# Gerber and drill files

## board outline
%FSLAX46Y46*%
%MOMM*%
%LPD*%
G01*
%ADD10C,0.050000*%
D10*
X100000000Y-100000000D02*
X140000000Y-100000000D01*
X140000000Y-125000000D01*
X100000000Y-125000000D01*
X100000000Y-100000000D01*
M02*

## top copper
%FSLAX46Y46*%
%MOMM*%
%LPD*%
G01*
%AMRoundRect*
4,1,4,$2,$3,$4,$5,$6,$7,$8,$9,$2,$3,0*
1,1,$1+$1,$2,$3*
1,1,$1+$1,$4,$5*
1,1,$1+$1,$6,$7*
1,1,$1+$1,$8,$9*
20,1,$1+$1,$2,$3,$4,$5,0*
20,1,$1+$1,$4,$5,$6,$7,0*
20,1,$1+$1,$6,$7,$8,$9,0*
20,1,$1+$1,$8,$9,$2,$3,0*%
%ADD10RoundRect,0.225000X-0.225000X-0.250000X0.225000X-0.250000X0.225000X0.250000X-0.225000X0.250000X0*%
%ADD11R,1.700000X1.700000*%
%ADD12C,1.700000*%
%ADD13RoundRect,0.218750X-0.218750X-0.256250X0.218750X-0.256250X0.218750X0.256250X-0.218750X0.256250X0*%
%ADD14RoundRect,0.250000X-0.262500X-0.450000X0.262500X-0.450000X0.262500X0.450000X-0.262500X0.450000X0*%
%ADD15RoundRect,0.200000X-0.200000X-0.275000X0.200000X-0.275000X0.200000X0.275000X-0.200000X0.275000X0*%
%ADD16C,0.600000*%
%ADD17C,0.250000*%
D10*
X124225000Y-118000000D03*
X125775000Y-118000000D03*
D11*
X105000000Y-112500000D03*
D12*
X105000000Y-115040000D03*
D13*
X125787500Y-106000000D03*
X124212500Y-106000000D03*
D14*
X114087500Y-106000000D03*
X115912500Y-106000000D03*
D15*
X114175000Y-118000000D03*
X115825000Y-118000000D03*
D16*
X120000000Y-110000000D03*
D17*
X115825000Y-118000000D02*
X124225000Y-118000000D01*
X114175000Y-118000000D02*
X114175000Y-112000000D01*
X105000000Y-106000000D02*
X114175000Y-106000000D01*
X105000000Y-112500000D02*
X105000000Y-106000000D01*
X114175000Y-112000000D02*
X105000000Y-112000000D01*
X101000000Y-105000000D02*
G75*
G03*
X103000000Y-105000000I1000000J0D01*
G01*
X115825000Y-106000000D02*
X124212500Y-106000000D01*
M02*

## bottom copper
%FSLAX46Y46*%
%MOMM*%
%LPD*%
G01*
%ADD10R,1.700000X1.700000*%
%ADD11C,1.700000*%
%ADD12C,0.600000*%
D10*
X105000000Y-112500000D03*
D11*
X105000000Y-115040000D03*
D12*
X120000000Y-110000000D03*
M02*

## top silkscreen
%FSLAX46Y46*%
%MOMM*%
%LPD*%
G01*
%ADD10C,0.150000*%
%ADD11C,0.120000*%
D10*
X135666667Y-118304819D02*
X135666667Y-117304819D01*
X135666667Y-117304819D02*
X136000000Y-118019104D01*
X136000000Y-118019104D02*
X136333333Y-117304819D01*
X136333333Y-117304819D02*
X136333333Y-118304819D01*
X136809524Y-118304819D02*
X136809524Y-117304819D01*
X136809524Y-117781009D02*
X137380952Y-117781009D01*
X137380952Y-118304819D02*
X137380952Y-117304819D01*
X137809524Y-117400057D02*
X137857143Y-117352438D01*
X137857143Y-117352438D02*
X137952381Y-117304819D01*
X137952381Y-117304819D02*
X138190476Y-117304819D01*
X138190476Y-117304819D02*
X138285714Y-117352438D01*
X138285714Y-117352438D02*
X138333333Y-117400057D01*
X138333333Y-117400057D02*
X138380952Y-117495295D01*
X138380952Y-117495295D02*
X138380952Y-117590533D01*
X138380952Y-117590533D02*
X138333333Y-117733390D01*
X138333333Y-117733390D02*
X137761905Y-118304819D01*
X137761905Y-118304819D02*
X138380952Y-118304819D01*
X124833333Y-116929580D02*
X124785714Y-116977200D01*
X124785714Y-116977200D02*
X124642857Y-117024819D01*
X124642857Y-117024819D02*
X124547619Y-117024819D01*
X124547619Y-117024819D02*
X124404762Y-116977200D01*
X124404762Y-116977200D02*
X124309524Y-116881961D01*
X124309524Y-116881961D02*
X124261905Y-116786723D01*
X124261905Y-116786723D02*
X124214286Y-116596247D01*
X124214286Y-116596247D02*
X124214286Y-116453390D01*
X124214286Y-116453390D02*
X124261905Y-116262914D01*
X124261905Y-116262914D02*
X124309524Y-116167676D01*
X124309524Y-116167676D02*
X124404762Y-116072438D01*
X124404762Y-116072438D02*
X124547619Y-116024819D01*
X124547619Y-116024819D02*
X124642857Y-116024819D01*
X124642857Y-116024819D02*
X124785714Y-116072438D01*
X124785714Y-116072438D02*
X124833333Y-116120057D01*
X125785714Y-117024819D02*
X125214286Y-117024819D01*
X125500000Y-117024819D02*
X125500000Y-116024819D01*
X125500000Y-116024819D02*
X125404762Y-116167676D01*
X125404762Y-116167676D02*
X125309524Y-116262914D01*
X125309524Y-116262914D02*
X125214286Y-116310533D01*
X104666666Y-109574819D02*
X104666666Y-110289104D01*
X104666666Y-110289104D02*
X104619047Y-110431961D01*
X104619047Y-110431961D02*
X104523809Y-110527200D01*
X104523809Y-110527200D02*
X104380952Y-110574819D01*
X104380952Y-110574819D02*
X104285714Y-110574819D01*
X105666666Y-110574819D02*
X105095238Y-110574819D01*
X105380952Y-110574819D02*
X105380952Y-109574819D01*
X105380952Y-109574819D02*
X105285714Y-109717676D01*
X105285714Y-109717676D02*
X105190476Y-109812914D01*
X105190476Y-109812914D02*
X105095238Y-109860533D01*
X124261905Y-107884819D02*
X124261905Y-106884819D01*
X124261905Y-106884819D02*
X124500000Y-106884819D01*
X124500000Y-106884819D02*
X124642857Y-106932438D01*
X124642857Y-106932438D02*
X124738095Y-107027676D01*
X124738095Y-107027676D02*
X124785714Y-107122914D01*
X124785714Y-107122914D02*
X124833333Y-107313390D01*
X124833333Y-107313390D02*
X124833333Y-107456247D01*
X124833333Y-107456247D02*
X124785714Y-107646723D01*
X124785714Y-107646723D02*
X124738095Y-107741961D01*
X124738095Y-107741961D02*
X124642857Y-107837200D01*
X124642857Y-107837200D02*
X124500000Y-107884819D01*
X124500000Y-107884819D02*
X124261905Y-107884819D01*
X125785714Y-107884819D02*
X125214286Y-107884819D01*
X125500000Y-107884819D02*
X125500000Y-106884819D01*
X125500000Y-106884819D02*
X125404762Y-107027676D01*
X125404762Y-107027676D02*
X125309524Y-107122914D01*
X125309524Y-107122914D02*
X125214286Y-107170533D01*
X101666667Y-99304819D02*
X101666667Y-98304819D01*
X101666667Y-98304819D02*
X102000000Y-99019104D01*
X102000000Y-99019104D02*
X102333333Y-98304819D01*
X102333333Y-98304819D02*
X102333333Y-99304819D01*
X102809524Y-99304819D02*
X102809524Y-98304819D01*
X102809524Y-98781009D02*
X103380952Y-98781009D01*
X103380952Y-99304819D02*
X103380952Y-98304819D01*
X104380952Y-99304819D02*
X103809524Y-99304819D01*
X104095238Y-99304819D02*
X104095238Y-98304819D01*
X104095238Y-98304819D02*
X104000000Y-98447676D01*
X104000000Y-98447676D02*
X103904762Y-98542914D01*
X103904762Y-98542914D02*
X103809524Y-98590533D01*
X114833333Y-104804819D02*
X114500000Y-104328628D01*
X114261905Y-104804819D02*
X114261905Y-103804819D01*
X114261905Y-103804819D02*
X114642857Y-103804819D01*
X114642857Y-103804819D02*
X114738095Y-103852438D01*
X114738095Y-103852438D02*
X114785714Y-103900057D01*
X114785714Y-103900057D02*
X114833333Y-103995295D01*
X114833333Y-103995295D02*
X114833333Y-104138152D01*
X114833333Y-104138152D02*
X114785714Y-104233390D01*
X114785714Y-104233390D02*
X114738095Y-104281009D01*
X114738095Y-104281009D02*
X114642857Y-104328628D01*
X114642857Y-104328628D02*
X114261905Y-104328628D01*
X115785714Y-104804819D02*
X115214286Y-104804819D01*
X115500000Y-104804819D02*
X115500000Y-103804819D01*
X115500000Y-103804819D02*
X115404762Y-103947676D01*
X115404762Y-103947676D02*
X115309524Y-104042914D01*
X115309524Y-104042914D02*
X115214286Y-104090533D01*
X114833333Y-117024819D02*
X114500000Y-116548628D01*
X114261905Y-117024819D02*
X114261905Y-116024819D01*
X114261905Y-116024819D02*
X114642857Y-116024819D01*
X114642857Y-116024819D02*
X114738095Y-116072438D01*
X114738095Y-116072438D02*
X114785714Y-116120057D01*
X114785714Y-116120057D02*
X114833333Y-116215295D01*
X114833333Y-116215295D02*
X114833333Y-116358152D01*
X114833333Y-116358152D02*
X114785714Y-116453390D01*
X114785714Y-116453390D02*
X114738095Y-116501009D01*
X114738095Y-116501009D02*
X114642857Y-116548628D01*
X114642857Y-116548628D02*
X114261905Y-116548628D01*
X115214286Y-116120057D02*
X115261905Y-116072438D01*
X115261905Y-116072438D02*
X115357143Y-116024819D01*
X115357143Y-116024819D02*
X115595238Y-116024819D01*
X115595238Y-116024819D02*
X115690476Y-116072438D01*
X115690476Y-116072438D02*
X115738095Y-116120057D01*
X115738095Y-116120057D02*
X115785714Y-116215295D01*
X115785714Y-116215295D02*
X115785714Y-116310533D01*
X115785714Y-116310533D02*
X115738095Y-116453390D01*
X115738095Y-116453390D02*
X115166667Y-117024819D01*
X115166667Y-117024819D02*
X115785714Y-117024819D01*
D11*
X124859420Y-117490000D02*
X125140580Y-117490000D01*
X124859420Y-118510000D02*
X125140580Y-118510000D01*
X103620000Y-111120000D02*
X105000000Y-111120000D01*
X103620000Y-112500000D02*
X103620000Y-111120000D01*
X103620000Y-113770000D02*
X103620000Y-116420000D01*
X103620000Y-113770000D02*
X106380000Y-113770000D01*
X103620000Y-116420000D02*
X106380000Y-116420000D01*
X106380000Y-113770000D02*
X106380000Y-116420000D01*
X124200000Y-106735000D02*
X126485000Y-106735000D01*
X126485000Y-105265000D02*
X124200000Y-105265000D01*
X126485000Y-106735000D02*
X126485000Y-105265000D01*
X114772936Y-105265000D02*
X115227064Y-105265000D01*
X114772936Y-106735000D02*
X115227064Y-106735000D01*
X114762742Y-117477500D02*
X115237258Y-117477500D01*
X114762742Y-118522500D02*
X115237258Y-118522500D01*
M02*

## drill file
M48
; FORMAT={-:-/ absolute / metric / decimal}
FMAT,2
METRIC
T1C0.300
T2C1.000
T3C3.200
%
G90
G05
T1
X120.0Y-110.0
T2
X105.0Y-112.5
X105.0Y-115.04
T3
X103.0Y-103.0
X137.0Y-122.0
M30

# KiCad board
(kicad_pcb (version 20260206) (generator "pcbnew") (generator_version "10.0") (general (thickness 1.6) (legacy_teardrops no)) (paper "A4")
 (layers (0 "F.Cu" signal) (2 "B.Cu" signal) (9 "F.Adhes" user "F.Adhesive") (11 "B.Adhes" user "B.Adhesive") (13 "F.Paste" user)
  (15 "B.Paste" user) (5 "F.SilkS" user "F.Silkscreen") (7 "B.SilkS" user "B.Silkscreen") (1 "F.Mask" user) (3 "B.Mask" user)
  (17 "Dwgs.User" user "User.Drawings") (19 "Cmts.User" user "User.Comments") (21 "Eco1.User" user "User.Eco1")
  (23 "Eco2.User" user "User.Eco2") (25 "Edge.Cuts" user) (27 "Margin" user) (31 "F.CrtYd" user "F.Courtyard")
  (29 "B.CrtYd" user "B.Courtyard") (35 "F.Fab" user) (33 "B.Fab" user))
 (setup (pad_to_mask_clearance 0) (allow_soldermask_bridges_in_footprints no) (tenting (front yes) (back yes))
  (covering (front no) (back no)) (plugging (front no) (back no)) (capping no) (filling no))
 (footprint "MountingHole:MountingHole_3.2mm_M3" (layer "F.Cu") (at 137 122)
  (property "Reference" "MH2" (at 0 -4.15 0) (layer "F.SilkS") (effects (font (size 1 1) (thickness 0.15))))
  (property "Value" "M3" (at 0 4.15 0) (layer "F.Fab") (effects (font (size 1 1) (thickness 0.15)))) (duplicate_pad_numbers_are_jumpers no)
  (pad "" np_thru_hole circle (at 0 0) (size 3.2 3.2) (drill 3.2) (layers "*.Cu" "*.Mask")))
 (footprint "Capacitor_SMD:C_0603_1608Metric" (layer "F.Cu") (at 125 118)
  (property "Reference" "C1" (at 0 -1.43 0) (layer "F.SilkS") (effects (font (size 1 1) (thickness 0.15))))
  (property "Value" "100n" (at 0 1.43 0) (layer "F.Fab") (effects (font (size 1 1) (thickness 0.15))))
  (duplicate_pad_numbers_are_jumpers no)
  (fp_line (start -0.14058 -0.51) (end 0.14058 -0.51) (stroke (width 0.12) (type solid)) (layer "F.SilkS"))
  (fp_line (start -0.14058 0.51) (end 0.14058 0.51) (stroke (width 0.12) (type solid)) (layer "F.SilkS"))
  (pad "1" smd roundrect (at -0.775 0) (size 0.9 0.95) (layers "F.Cu" "F.Mask" "F.Paste") (roundrect_rratio 0.25) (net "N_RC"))
  (pad "2" smd roundrect (at 0.775 0) (size 0.9 0.95) (layers "F.Cu" "F.Mask" "F.Paste") (roundrect_rratio 0.25) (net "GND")))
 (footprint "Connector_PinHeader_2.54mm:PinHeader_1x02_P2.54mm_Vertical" (layer "F.Cu") (at 105 112.5)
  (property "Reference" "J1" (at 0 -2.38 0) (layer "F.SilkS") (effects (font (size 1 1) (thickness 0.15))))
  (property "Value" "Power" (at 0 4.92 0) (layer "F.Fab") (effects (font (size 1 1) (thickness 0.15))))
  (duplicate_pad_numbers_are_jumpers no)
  (fp_line (start -1.38 -1.38) (end 0 -1.38) (stroke (width 0.12) (type solid)) (layer "F.SilkS"))
  (fp_line (start -1.38 0) (end -1.38 -1.38) (stroke (width 0.12) (type solid)) (layer "F.SilkS"))
  (fp_line (start -1.38 1.27) (end -1.38 3.92) (stroke (width 0.12) (type solid)) (layer "F.SilkS"))
  (fp_line (start -1.38 1.27) (end 1.38 1.27) (stroke (width 0.12) (type solid)) (layer "F.SilkS"))
  (fp_line (start -1.38 3.92) (end 1.38 3.92) (stroke (width 0.12) (type solid)) (layer "F.SilkS"))
  (fp_line (start 1.38 1.27) (end 1.38 3.92) (stroke (width 0.12) (type solid)) (layer "F.SilkS"))
  (pad "1" thru_hole rect (at 0 0) (size 1.7 1.7) (drill 1) (layers "*.Cu" "*.Mask") (remove_unused_layers no) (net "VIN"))
  (pad "2" thru_hole circle (at 0 2.54) (size 1.7 1.7) (drill 1) (layers "*.Cu" "*.Mask") (remove_unused_layers no) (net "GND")))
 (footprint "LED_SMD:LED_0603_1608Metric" (layer "F.Cu") (at 125 106 180)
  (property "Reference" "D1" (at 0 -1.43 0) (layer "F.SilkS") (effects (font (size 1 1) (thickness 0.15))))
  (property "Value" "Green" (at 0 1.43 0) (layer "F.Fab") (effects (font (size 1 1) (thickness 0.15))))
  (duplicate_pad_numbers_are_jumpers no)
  (fp_line (start 0.8 -0.735) (end -1.485 -0.735) (stroke (width 0.12) (type solid)) (layer "F.SilkS"))
  (fp_line (start -1.485 0.735) (end 0.8 0.735) (stroke (width 0.12) (type solid)) (layer "F.SilkS"))
  (fp_line (start -1.485 -0.735) (end -1.485 0.735) (stroke (width 0.12) (type solid)) (layer "F.SilkS"))
  (pad "1" smd roundrect (at -0.7875 0) (size 0.875 0.95) (layers "F.Cu" "F.Mask" "F.Paste") (roundrect_rratio 0.25) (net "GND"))
  (pad "2" smd roundrect (at 0.7875 0) (size 0.875 0.95) (layers "F.Cu" "F.Mask" "F.Paste") (roundrect_rratio 0.25) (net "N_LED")))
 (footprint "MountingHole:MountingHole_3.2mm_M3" (layer "F.Cu") (at 103 103)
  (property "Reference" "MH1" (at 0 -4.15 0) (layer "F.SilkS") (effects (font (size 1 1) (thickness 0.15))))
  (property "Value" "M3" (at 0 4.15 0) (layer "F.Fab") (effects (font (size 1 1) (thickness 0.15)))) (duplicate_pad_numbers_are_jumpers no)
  (pad "" np_thru_hole circle (at 0 0) (size 3.2 3.2) (drill 3.2) (layers "*.Cu" "*.Mask")))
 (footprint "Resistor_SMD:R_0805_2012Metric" (layer "F.Cu") (at 115 106)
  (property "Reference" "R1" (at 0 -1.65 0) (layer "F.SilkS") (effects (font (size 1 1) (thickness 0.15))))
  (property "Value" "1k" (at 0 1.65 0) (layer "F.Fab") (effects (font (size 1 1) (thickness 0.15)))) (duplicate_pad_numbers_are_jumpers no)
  (fp_line (start -0.227064 -0.735) (end 0.227064 -0.735) (stroke (width 0.12) (type solid)) (layer "F.SilkS"))
  (fp_line (start -0.227064 0.735) (end 0.227064 0.735) (stroke (width 0.12) (type solid)) (layer "F.SilkS"))
  (pad "1" smd roundrect (at -0.9125 0) (size 1.025 1.4) (layers "F.Cu" "F.Mask" "F.Paste") (roundrect_rratio 0.243902) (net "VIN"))
  (pad "2" smd roundrect (at 0.9125 0) (size 1.025 1.4) (layers "F.Cu" "F.Mask" "F.Paste") (roundrect_rratio 0.243902) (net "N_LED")))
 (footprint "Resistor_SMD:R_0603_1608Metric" (layer "F.Cu") (at 115 118)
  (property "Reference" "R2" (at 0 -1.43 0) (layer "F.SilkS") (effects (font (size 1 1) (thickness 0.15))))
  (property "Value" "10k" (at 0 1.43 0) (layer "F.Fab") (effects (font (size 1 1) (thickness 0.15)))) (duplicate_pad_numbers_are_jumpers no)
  (fp_line (start -0.237258 -0.5225) (end 0.237258 -0.5225) (stroke (width 0.12) (type solid)) (layer "F.SilkS"))
  (fp_line (start -0.237258 0.5225) (end 0.237258 0.5225) (stroke (width 0.12) (type solid)) (layer "F.SilkS"))
  (pad "1" smd roundrect (at -0.825 0) (size 0.8 0.95) (layers "F.Cu" "F.Mask" "F.Paste") (roundrect_rratio 0.25) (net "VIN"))
  (pad "2" smd roundrect (at 0.825 0) (size 0.8 0.95) (layers "F.Cu" "F.Mask" "F.Paste") (roundrect_rratio 0.25) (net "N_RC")))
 (gr_rect (start 100 100) (end 140 125) (stroke (width 0.05) (type default)) (fill no) (layer "Edge.Cuts"))
 (segment (start 115.825 118) (end 124.225 118) (width 0.25) (layer "F.Cu") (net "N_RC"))
 (segment (start 114.175 118) (end 114.175 112) (width 0.25) (layer "F.Cu") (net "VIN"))
 (segment (start 105 106) (end 114.175 106) (width 0.25) (layer "F.Cu") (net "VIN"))
 (segment (start 105 112.5) (end 105 106) (width 0.25) (layer "F.Cu") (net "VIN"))
 (segment (start 114.175 112) (end 105 112) (width 0.25) (layer "F.Cu") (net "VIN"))
 (via (at 120 110) (size 0.6) (drill 0.3) (layers "F.Cu" "B.Cu") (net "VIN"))
 (arc (start 101 105) (mid 102 106) (end 103 105) (width 0.25) (layer "F.Cu") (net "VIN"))
 (segment (start 115.825 106) (end 124.2125 106) (width 0.25) (layer "F.Cu") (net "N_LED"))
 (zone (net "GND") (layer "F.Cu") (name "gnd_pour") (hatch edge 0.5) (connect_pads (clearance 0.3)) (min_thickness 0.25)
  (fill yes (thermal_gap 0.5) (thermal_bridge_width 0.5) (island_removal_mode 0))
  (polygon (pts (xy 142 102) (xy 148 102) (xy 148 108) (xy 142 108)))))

